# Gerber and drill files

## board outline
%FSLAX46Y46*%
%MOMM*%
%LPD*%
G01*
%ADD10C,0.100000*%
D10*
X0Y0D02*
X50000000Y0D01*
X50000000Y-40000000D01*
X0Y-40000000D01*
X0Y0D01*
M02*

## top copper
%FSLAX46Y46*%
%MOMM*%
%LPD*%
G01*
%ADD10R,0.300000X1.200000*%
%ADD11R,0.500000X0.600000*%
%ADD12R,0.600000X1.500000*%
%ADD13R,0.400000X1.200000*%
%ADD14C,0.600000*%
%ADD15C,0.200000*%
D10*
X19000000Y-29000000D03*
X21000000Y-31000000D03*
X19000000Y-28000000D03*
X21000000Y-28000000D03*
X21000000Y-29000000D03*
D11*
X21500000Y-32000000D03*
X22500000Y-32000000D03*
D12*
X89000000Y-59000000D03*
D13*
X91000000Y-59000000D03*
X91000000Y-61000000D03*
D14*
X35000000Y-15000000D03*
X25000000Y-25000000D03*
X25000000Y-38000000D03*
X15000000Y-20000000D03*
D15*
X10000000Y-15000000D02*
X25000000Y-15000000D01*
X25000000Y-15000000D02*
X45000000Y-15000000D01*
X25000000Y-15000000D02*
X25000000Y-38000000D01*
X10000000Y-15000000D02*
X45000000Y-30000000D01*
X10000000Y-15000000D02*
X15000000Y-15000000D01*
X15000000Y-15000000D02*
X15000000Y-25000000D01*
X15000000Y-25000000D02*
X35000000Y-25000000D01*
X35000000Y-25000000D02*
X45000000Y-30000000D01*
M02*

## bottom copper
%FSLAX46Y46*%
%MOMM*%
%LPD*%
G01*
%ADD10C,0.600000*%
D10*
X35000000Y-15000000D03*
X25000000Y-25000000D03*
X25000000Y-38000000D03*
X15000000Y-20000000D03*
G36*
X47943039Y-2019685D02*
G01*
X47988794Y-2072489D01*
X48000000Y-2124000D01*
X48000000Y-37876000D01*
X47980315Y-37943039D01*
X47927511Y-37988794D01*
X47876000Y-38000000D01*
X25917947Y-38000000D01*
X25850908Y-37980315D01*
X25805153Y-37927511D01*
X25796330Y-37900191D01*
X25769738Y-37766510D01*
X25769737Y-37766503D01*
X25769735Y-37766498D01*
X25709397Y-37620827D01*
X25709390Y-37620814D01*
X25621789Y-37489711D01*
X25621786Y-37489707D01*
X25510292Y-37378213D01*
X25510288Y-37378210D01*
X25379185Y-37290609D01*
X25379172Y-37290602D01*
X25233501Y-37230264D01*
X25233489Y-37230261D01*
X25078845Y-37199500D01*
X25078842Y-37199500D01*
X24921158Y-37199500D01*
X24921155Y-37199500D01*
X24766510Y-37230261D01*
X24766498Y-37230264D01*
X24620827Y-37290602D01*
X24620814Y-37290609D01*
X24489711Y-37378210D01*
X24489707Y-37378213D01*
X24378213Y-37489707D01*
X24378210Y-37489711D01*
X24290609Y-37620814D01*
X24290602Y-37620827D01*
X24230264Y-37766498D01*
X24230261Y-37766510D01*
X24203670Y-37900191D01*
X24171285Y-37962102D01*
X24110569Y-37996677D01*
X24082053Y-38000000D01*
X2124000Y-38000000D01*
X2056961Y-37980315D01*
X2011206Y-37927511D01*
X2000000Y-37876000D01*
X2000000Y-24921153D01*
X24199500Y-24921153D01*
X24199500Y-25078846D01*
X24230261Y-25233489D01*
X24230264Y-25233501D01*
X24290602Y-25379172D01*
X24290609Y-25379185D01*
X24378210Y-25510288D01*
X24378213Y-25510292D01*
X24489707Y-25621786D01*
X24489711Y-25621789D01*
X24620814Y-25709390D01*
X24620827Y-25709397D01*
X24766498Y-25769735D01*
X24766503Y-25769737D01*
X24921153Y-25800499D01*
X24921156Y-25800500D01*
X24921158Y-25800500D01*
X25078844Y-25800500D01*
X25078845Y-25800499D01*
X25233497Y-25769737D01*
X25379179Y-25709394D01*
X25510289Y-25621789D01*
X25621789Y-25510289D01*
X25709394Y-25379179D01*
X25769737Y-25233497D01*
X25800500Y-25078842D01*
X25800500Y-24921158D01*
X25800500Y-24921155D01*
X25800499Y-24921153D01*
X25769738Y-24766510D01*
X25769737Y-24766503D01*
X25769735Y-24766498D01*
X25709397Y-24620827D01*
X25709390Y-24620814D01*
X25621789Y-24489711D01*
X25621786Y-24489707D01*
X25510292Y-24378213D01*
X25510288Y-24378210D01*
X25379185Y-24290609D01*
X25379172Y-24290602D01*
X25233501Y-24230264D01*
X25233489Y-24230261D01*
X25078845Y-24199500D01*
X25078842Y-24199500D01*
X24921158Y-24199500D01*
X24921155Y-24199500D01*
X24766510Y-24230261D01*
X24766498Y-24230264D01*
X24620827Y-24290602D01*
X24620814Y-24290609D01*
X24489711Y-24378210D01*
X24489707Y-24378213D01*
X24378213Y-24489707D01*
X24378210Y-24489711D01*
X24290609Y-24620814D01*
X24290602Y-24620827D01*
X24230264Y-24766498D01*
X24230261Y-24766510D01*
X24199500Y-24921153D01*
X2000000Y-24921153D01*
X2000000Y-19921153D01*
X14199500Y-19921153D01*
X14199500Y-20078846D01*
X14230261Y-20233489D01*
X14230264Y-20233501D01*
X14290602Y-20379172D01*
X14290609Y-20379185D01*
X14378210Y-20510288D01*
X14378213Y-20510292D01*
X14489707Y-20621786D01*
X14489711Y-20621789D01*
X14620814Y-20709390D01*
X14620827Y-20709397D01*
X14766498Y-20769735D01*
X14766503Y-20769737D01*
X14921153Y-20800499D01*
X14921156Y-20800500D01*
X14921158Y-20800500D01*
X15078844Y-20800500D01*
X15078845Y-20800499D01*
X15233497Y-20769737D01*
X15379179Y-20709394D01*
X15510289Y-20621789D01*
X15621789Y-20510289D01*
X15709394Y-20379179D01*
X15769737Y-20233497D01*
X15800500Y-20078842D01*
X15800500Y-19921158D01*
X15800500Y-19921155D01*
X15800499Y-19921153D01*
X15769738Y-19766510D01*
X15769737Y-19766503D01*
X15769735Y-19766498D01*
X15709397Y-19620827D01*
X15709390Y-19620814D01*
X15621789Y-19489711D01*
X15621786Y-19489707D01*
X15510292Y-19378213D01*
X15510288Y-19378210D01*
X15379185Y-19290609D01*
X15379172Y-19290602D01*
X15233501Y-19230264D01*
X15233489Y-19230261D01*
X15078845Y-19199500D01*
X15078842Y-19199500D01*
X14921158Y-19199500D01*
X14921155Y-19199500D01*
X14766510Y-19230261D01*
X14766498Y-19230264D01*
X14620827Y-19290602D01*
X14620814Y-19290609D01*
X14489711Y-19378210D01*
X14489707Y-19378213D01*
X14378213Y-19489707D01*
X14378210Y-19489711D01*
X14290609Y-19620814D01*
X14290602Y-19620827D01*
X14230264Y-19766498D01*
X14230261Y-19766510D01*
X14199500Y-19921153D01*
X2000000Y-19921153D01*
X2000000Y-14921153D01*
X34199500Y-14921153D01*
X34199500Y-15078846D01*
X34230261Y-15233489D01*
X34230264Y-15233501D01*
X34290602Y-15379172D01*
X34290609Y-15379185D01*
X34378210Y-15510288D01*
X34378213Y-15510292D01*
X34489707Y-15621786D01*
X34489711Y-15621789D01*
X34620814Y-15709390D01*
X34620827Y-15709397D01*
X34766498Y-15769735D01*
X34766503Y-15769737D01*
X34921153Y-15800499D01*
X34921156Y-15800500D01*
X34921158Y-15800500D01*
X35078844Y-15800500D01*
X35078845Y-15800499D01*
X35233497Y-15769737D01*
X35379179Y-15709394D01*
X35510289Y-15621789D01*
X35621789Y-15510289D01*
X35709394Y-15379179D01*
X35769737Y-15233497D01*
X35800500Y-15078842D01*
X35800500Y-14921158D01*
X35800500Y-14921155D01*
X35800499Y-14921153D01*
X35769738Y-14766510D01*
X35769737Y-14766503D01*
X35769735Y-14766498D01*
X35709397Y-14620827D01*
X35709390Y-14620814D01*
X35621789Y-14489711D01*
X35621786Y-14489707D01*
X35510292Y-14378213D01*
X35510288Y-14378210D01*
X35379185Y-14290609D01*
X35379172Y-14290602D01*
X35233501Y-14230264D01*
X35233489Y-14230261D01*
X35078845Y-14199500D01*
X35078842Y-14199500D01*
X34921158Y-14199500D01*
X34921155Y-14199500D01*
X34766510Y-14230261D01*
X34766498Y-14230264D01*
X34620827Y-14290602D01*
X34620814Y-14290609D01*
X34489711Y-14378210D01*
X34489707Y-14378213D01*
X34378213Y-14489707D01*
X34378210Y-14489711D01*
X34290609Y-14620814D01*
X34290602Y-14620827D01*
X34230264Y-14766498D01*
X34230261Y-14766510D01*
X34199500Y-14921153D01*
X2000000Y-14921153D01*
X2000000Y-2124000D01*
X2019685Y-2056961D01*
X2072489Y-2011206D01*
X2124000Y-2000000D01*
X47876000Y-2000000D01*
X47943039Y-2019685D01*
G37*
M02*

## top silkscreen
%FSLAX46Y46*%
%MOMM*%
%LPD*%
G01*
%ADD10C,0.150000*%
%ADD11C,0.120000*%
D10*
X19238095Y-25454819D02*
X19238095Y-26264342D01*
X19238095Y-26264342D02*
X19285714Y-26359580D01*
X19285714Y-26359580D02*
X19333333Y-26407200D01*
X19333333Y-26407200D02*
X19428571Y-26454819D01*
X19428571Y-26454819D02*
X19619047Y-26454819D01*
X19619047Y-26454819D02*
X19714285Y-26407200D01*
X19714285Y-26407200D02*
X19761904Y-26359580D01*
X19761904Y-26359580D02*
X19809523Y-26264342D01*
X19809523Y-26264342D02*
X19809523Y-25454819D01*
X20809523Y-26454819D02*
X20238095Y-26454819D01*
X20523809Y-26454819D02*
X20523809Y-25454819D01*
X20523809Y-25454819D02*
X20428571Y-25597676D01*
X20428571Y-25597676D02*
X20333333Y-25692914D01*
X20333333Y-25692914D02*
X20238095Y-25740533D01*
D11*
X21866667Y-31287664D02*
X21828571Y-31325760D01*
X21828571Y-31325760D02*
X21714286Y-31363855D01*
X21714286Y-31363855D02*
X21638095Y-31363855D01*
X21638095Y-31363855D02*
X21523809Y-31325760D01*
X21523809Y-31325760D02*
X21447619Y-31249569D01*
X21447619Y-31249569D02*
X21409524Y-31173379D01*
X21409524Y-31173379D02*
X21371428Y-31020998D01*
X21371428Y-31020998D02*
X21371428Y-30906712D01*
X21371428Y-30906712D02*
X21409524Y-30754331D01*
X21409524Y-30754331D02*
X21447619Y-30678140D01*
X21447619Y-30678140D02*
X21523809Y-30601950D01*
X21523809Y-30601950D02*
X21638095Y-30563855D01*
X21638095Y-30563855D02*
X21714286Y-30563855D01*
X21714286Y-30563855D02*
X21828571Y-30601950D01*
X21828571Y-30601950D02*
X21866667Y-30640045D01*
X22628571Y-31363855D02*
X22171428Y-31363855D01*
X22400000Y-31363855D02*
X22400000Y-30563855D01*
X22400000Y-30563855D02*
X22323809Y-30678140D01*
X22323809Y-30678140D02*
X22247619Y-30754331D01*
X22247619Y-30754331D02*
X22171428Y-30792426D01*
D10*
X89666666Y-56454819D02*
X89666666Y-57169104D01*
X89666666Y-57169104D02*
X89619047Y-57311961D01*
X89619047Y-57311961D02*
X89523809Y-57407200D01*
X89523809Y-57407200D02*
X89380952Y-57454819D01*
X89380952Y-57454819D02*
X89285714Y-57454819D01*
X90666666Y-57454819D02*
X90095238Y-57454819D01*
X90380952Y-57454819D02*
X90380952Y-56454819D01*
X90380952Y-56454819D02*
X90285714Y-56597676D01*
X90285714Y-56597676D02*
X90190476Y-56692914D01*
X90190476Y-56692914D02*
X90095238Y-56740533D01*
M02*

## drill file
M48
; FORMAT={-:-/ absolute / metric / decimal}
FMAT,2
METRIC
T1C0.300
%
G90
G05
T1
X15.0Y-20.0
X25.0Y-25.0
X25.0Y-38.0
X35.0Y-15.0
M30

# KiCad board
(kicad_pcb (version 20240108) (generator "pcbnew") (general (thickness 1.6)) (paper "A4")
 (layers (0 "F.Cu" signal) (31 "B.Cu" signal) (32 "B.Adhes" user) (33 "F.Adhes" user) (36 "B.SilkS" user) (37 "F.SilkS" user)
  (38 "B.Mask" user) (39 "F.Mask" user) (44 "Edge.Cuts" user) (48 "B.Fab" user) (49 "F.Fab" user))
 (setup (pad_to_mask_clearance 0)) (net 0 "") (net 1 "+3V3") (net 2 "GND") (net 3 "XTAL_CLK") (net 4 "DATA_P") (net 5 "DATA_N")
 (gr_rect (start 0 0) (end 50 40) (layer "Edge.Cuts") (width 0.1))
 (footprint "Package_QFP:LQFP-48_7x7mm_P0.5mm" (layer "F.Cu") (at 10 15 0)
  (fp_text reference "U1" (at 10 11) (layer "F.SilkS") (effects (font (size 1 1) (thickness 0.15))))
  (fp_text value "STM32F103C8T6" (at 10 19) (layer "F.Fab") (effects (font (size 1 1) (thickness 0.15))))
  (pad "8" smd rect (at 9 14) (size 0.3 1.2) (layers "F.Cu" "F.Paste" "F.Mask") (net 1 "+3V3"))
  (pad "23" smd rect (at 11 16) (size 0.3 1.2) (layers "F.Cu" "F.Paste" "F.Mask") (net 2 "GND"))
  (pad "5" smd rect (at 9 13) (size 0.3 1.2) (layers "F.Cu" "F.Paste" "F.Mask") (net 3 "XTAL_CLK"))
  (pad "44" smd rect (at 11 13) (size 0.3 1.2) (layers "F.Cu" "F.Paste" "F.Mask") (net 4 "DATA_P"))
  (pad "43" smd rect (at 11 14) (size 0.3 1.2) (layers "F.Cu" "F.Paste" "F.Mask") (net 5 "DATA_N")))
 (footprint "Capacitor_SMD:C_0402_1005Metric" (layer "F.Cu") (at 11 16 0)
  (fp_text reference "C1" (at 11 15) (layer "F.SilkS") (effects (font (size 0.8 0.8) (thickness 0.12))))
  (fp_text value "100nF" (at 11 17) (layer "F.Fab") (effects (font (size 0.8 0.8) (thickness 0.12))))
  (pad "1" smd rect (at 10.5 16) (size 0.5 0.6) (layers "F.Cu" "F.Paste" "F.Mask") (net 1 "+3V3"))
  (pad "2" smd rect (at 11.5 16) (size 0.5 0.6) (layers "F.Cu" "F.Paste" "F.Mask") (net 2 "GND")))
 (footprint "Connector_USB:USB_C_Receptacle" (layer "F.Cu") (at 45 30 0)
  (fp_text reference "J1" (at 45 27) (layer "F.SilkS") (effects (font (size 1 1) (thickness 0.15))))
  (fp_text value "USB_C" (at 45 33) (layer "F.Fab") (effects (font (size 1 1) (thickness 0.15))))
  (pad "GND" smd rect (at 44 29) (size 0.6 1.5) (layers "F.Cu" "F.Paste" "F.Mask") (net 2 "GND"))
  (pad "DP" smd rect (at 46 29) (size 0.4 1.2) (layers "F.Cu" "F.Paste" "F.Mask") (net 4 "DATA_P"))
  (pad "DM" smd rect (at 46 31) (size 0.4 1.2) (layers "F.Cu" "F.Paste" "F.Mask") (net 5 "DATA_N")))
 (segment (start 10 15) (end 25 15) (width 0.2) (layer "F.Cu") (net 3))
 (segment (start 25 15) (end 45 15) (width 0.2) (layer "F.Cu") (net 3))
 (segment (start 25 15) (end 25 38) (width 0.2) (layer "F.Cu") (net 3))
 (via (at 35 15) (size 0.6) (drill 0.3) (layers "F.Cu" "B.Cu") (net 3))
 (via (at 25 25) (size 0.6) (drill 0.3) (layers "F.Cu" "B.Cu") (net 3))
 (via (at 25 38) (size 0.6) (drill 0.3) (layers "F.Cu" "B.Cu") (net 3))
 (segment (start 10 15) (end 45 30) (width 0.2) (layer "F.Cu") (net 4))
 (segment (start 10 15) (end 15 15) (width 0.2) (layer "F.Cu") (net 5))
 (segment (start 15 15) (end 15 25) (width 0.2) (layer "F.Cu") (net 5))
 (segment (start 15 25) (end 35 25) (width 0.2) (layer "F.Cu") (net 5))
 (segment (start 35 25) (end 45 30) (width 0.2) (layer "F.Cu") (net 5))
 (via (at 15 20) (size 0.6) (drill 0.3) (layers "F.Cu" "B.Cu") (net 5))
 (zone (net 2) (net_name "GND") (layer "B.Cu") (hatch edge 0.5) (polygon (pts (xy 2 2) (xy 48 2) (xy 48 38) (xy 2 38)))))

